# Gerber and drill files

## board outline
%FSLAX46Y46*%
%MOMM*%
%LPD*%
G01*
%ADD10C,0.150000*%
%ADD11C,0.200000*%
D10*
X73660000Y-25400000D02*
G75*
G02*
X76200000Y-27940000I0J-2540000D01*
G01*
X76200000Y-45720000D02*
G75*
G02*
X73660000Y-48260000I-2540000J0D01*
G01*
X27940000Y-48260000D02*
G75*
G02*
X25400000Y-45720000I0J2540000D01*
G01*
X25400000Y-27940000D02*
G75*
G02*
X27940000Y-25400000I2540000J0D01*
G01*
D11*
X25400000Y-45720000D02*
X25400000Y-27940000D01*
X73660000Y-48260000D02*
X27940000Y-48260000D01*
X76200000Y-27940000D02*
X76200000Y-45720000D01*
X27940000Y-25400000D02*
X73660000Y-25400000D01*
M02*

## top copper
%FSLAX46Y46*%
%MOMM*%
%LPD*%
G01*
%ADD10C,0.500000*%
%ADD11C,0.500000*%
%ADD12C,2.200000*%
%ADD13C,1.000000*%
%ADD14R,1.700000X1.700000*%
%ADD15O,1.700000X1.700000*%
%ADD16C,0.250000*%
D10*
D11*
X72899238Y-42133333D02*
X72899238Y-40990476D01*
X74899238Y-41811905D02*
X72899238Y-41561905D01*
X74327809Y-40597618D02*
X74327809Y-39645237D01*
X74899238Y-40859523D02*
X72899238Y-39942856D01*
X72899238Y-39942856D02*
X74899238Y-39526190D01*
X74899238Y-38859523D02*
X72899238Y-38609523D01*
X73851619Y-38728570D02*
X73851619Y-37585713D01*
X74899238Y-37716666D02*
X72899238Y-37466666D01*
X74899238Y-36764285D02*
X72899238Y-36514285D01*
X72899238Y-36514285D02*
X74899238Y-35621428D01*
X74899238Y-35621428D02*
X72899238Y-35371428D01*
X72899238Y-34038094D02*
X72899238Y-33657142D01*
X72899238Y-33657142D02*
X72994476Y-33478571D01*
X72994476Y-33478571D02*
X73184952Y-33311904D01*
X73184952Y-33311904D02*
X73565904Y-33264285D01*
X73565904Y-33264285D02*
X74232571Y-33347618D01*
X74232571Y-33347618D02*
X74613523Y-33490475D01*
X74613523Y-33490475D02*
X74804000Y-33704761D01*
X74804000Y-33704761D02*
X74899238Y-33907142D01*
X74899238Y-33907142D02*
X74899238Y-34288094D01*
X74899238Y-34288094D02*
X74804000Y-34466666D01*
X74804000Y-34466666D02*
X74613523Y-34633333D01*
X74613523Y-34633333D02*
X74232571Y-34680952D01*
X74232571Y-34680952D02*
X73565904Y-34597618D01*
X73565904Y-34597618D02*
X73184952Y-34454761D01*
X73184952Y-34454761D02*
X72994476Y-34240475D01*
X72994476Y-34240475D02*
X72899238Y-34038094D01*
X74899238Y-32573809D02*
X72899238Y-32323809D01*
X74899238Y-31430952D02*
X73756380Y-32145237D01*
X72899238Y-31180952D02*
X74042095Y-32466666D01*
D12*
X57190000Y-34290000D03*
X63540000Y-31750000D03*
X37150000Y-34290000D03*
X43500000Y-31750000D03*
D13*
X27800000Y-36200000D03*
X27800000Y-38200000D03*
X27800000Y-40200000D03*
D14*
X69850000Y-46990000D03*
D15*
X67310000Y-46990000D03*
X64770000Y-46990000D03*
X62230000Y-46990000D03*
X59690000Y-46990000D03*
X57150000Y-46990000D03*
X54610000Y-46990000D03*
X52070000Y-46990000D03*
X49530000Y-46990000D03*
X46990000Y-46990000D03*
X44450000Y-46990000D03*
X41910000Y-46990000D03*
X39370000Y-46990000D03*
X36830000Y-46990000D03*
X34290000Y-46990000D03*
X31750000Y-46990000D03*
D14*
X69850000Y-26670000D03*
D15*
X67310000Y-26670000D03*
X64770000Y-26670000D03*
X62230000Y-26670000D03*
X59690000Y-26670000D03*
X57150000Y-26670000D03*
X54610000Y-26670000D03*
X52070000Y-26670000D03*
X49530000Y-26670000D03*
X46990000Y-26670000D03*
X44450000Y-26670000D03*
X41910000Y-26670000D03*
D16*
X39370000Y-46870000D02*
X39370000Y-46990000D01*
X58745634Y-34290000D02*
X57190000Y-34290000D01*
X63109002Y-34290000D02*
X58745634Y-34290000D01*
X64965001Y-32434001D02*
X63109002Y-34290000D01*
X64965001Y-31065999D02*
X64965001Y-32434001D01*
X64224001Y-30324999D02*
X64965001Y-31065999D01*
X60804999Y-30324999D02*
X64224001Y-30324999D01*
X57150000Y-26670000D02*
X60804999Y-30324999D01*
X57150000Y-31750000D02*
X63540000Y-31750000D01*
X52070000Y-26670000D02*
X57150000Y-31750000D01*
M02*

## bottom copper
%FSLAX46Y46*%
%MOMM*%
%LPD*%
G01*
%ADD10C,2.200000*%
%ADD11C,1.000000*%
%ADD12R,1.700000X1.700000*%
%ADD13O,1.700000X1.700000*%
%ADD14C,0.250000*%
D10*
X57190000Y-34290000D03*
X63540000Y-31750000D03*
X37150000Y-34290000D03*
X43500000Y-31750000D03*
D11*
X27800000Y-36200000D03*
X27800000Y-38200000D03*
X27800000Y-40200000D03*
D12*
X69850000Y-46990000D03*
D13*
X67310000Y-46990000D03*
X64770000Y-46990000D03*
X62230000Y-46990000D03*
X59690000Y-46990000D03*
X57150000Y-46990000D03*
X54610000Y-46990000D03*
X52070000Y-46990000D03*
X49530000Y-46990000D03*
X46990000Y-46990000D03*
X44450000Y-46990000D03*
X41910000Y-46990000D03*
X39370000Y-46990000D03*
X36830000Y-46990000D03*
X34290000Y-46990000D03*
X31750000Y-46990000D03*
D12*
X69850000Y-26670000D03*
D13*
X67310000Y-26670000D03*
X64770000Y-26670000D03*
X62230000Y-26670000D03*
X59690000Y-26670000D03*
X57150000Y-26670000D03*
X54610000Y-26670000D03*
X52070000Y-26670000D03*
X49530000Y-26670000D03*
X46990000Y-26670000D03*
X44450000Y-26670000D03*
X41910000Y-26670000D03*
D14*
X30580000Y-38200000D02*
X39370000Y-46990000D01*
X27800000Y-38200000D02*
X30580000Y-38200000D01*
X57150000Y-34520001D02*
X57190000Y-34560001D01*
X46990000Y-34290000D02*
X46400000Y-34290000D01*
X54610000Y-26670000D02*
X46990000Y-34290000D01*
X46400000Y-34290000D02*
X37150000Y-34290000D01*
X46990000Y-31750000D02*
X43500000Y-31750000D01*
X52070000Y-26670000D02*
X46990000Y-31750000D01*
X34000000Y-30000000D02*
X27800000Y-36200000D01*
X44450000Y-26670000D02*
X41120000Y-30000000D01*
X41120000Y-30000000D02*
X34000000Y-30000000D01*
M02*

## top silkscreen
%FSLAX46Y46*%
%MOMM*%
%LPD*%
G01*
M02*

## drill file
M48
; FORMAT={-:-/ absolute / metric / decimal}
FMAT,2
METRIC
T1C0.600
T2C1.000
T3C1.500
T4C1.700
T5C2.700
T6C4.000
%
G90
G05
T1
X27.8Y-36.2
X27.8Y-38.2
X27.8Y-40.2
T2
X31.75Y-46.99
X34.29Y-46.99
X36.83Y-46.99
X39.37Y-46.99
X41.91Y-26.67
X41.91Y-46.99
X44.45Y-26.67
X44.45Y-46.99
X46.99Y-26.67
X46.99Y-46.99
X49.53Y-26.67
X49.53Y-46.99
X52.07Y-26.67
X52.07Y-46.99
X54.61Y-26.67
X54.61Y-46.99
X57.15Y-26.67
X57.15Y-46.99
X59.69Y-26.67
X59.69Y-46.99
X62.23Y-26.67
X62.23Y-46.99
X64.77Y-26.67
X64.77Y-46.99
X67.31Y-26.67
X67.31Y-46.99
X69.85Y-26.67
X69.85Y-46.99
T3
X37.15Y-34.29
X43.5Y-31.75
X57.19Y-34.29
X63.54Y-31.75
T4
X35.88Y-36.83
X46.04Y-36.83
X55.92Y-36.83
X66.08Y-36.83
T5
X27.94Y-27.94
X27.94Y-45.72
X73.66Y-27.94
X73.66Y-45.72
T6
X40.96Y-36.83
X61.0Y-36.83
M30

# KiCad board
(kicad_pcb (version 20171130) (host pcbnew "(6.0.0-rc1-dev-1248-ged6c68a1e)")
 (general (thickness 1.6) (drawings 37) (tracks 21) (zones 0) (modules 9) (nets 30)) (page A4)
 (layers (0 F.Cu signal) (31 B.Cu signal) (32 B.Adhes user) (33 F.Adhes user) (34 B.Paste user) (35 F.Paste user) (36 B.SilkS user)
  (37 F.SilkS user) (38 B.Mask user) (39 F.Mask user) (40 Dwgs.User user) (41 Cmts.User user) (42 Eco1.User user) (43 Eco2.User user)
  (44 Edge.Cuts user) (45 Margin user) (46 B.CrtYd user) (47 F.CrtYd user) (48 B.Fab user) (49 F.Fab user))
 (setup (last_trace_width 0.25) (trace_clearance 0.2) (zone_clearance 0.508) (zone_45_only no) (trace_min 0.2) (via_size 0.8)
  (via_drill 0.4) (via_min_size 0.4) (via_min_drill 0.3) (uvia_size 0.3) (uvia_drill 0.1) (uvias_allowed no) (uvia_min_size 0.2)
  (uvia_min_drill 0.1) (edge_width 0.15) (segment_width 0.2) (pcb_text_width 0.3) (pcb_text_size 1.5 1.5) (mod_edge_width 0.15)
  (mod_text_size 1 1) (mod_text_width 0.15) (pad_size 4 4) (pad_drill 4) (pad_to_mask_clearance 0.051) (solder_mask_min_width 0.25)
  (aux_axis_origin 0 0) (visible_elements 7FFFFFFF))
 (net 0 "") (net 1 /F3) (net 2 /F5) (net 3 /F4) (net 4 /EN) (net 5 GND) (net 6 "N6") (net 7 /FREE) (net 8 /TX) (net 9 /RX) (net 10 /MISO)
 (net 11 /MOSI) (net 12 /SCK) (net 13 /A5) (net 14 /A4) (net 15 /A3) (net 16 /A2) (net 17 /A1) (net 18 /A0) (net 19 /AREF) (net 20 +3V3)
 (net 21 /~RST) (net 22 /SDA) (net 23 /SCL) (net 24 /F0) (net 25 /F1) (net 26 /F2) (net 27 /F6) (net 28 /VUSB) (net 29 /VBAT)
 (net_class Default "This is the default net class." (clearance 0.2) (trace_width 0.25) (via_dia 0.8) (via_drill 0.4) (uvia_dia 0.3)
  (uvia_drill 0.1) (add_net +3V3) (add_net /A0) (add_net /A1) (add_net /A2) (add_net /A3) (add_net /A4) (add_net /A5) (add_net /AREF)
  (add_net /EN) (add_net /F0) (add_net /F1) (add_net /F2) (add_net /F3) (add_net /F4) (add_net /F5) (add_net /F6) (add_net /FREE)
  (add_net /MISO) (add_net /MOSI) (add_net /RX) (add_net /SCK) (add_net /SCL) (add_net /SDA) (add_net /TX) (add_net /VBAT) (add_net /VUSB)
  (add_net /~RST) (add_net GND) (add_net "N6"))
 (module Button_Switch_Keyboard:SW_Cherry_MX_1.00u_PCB (layer F.Cu) (at 63.54 31.75)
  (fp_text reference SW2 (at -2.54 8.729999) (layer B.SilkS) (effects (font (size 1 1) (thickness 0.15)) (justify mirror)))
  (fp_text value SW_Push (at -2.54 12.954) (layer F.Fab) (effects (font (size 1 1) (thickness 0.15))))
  (pad "" np_thru_hole circle (at 2.54 5.08) (size 1.7 1.7) (drill 1.7) (layers *.Cu *.Mask))
  (pad "" np_thru_hole circle (at -7.62 5.08) (size 1.7 1.7) (drill 1.7) (layers *.Cu *.Mask))
  (pad "" np_thru_hole circle (at -2.54 5.08) (size 4 4) (drill 4) (layers *.Cu *.Mask))
  (pad 2 thru_hole circle (at -6.35 2.54) (size 2.2 2.2) (drill 1.5) (layers *.Cu *.Mask) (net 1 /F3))
  (pad 1 thru_hole circle (at 0 0) (size 2.2 2.2) (drill 1.5) (layers *.Cu *.Mask) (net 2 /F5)))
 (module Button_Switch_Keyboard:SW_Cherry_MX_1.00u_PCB (layer F.Cu) (at 43.5 31.75)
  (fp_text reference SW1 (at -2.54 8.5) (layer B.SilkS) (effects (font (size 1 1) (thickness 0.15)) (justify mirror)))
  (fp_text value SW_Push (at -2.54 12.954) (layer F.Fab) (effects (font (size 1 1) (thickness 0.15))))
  (pad "" np_thru_hole circle (at 2.54 5.08) (size 1.7 1.7) (drill 1.7) (layers *.Cu *.Mask))
  (pad "" np_thru_hole circle (at -7.62 5.08) (size 1.7 1.7) (drill 1.7) (layers *.Cu *.Mask))
  (pad "" np_thru_hole circle (at -2.54 5.08) (size 4 4) (drill 4) (layers *.Cu *.Mask))
  (pad 2 thru_hole circle (at -6.35 2.54) (size 2.2 2.2) (drill 1.5) (layers *.Cu *.Mask) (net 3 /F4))
  (pad 1 thru_hole circle (at 0 0) (size 2.2 2.2) (drill 1.5) (layers *.Cu *.Mask) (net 2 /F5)))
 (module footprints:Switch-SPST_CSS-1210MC (layer B.Cu) (at 30.8 35.2 90)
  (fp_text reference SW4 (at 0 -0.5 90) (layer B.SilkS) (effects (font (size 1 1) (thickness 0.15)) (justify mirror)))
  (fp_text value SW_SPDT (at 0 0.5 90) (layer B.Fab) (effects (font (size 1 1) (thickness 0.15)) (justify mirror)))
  (pad 3 thru_hole circle (at -1 -3 90) (size 1 1) (drill 0.6) (layers *.Cu *.Mask) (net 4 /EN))
  (pad 2 thru_hole circle (at -3 -3 90) (size 1 1) (drill 0.6) (layers *.Cu *.Mask) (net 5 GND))
  (pad 1 thru_hole circle (at -5 -3 90) (size 1 1) (drill 0.6) (layers *.Cu *.Mask) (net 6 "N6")))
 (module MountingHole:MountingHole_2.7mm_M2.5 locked (layer F.Cu) (at 73.66 27.94)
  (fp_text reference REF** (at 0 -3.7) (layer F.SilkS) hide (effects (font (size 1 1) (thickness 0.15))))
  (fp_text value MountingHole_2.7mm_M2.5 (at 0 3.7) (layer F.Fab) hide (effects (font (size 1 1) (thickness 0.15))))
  (pad 1 np_thru_hole circle (at 0 0) (size 2.7 2.7) (drill 2.7) (layers *.Cu *.Mask)))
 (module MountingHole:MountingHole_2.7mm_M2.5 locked (layer F.Cu) (at 73.66 45.72)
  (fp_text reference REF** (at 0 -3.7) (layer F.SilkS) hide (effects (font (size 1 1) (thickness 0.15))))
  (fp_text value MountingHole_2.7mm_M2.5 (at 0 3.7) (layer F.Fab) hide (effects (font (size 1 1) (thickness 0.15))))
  (pad 1 np_thru_hole circle (at 0 0) (size 2.7 2.7) (drill 2.7) (layers *.Cu *.Mask)))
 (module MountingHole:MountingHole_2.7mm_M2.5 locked (layer F.Cu) (at 27.94 45.72)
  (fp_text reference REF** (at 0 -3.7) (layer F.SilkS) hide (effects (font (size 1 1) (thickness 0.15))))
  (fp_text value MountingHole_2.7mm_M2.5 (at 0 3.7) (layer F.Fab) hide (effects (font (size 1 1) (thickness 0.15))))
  (pad 1 np_thru_hole circle (at 0 0) (size 2.7 2.7) (drill 2.7) (layers *.Cu *.Mask)))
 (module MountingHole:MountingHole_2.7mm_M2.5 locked (layer F.Cu) (at 27.94 27.94)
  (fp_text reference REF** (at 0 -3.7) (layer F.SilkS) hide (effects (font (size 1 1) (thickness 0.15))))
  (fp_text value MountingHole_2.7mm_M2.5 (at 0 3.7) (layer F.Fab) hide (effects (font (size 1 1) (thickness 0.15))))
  (pad 1 np_thru_hole circle (at 0 0) (size 2.7 2.7) (drill 2.7) (layers *.Cu *.Mask)))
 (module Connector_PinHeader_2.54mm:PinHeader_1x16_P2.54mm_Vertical (layer B.Cu) (at 69.85 46.99 90)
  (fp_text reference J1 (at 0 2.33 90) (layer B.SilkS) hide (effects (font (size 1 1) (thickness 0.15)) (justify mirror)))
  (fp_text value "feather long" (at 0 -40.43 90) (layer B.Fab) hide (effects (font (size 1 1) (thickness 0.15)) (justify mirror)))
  (pad 1 thru_hole rect (at 0 0 90) (size 1.7 1.7) (drill 1) (layers *.Cu *.Mask) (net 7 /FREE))
  (pad 2 thru_hole oval (at 0 -2.54 90) (size 1.7 1.7) (drill 1) (layers *.Cu *.Mask) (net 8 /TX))
  (pad 3 thru_hole oval (at 0 -5.08 90) (size 1.7 1.7) (drill 1) (layers *.Cu *.Mask) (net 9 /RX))
  (pad 4 thru_hole oval (at 0 -7.62 90) (size 1.7 1.7) (drill 1) (layers *.Cu *.Mask) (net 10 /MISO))
  (pad 5 thru_hole oval (at 0 -10.16 90) (size 1.7 1.7) (drill 1) (layers *.Cu *.Mask) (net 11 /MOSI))
  (pad 6 thru_hole oval (at 0 -12.7 90) (size 1.7 1.7) (drill 1) (layers *.Cu *.Mask) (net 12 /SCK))
  (pad 7 thru_hole oval (at 0 -15.24 90) (size 1.7 1.7) (drill 1) (layers *.Cu *.Mask) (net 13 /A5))
  (pad 8 thru_hole oval (at 0 -17.78 90) (size 1.7 1.7) (drill 1) (layers *.Cu *.Mask) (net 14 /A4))
  (pad 9 thru_hole oval (at 0 -20.32 90) (size 1.7 1.7) (drill 1) (layers *.Cu *.Mask) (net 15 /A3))
  (pad 10 thru_hole oval (at 0 -22.86 90) (size 1.7 1.7) (drill 1) (layers *.Cu *.Mask) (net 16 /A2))
  (pad 11 thru_hole oval (at 0 -25.4 90) (size 1.7 1.7) (drill 1) (layers *.Cu *.Mask) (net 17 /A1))
  (pad 12 thru_hole oval (at 0 -27.94 90) (size 1.7 1.7) (drill 1) (layers *.Cu *.Mask) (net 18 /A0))
  (pad 13 thru_hole oval (at 0 -30.48 90) (size 1.7 1.7) (drill 1) (layers *.Cu *.Mask) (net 5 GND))
  (pad 14 thru_hole oval (at 0 -33.02 90) (size 1.7 1.7) (drill 1) (layers *.Cu *.Mask) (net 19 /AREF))
  (pad 15 thru_hole oval (at 0 -35.56 90) (size 1.7 1.7) (drill 1) (layers *.Cu *.Mask) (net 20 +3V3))
  (pad 16 thru_hole oval (at 0 -38.1 90) (size 1.7 1.7) (drill 1) (layers *.Cu *.Mask) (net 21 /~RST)))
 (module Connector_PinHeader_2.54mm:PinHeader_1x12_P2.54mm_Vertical (layer B.Cu) (at 69.85 26.67 90)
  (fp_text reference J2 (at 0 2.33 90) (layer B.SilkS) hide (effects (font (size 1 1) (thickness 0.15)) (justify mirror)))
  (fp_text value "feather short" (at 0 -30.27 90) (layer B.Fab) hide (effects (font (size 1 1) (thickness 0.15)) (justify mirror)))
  (pad 1 thru_hole rect (at 0 0 90) (size 1.7 1.7) (drill 1) (layers *.Cu *.Mask) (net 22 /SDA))
  (pad 2 thru_hole oval (at 0 -2.54 90) (size 1.7 1.7) (drill 1) (layers *.Cu *.Mask) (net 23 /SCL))
  (pad 3 thru_hole oval (at 0 -5.08 90) (size 1.7 1.7) (drill 1) (layers *.Cu *.Mask) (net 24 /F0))
  (pad 4 thru_hole oval (at 0 -7.62 90) (size 1.7 1.7) (drill 1) (layers *.Cu *.Mask) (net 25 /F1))
  (pad 5 thru_hole oval (at 0 -10.16 90) (size 1.7 1.7) (drill 1) (layers *.Cu *.Mask) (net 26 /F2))
  (pad 6 thru_hole oval (at 0 -12.7 90) (size 1.7 1.7) (drill 1) (layers *.Cu *.Mask) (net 1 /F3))
  (pad 7 thru_hole oval (at 0 -15.24 90) (size 1.7 1.7) (drill 1) (layers *.Cu *.Mask) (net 3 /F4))
  (pad 8 thru_hole oval (at 0 -17.78 90) (size 1.7 1.7) (drill 1) (layers *.Cu *.Mask) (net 2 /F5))
  (pad 9 thru_hole oval (at 0 -20.32 90) (size 1.7 1.7) (drill 1) (layers *.Cu *.Mask) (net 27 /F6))
  (pad 10 thru_hole oval (at 0 -22.86 90) (size 1.7 1.7) (drill 1) (layers *.Cu *.Mask) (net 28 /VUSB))
  (pad 11 thru_hole oval (at 0 -25.4 90) (size 1.7 1.7) (drill 1) (layers *.Cu *.Mask) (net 4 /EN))
  (pad 12 thru_hole oval (at 0 -27.94 90) (size 1.7 1.7) (drill 1) (layers *.Cu *.Mask) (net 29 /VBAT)))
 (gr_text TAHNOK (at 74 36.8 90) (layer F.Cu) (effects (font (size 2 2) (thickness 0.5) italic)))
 (gr_arc (start 73.66 27.94) (end 76.2 27.94) (angle -90) (layer Edge.Cuts) (width 0.15))
 (gr_arc (start 73.66 45.72) (end 73.66 48.26) (angle -90) (layer Edge.Cuts) (width 0.15))
 (gr_arc (start 27.94 45.72) (end 25.4 45.72) (angle -90) (layer Edge.Cuts) (width 0.15))
 (gr_arc (start 27.94 27.94) (end 27.94 25.4) (angle -90) (layer Edge.Cuts) (width 0.15))
 (gr_line (start 25.4 45.72) (end 25.4 27.94) (layer Edge.Cuts) (width 0.2))
 (gr_line (start 73.66 48.26) (end 27.94 48.26) (layer Edge.Cuts) (width 0.2))
 (gr_line (start 76.2 27.94) (end 76.2 45.72) (layer Edge.Cuts) (width 0.2))
 (gr_line (start 27.94 25.4) (end 73.66 25.4) (layer Edge.Cuts) (width 0.2))
 (segment (start 39.37 46.87) (end 39.37 46.99) (width 0.25) (layer F.Cu) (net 5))
 (segment (start 30.58 38.2) (end 39.37 46.99) (width 0.25) (layer B.Cu) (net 5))
 (segment (start 27.8 38.2) (end 30.58 38.2) (width 0.25) (layer B.Cu) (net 5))
 (segment (start 57.15 34.520001) (end 57.19 34.560001) (width 0.25) (layer B.Cu) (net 1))
 (segment (start 58.745634 34.29) (end 57.19 34.29) (width 0.25) (layer F.Cu) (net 1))
 (segment (start 63.109002 34.29) (end 58.745634 34.29) (width 0.25) (layer F.Cu) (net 1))
 (segment (start 64.965001 32.434001) (end 63.109002 34.29) (width 0.25) (layer F.Cu) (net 1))
 (segment (start 64.965001 31.065999) (end 64.965001 32.434001) (width 0.25) (layer F.Cu) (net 1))
 (segment (start 64.224001 30.324999) (end 64.965001 31.065999) (width 0.25) (layer F.Cu) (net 1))
 (segment (start 60.804999 30.324999) (end 64.224001 30.324999) (width 0.25) (layer F.Cu) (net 1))
 (segment (start 57.15 26.67) (end 60.804999 30.324999) (width 0.25) (layer F.Cu) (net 1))
 (segment (start 46.99 34.29) (end 46.4 34.29) (width 0.25) (layer B.Cu) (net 3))
 (segment (start 54.61 26.67) (end 46.99 34.29) (width 0.25) (layer B.Cu) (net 3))
 (segment (start 46.4 34.29) (end 37.15 34.29) (width 0.25) (layer B.Cu) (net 3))
 (segment (start 57.15 31.75) (end 63.54 31.75) (width 0.25) (layer F.Cu) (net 2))
 (segment (start 52.07 26.67) (end 57.15 31.75) (width 0.25) (layer F.Cu) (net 2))
 (segment (start 46.99 31.75) (end 43.5 31.75) (width 0.25) (layer B.Cu) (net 2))
 (segment (start 52.07 26.67) (end 46.99 31.75) (width 0.25) (layer B.Cu) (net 2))
 (segment (start 34 30) (end 27.8 36.2) (width 0.25) (layer B.Cu) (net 4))
 (segment (start 44.45 26.67) (end 41.12 30) (width 0.25) (layer B.Cu) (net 4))
 (segment (start 41.12 30) (end 34 30) (width 0.25) (layer B.Cu) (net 4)))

